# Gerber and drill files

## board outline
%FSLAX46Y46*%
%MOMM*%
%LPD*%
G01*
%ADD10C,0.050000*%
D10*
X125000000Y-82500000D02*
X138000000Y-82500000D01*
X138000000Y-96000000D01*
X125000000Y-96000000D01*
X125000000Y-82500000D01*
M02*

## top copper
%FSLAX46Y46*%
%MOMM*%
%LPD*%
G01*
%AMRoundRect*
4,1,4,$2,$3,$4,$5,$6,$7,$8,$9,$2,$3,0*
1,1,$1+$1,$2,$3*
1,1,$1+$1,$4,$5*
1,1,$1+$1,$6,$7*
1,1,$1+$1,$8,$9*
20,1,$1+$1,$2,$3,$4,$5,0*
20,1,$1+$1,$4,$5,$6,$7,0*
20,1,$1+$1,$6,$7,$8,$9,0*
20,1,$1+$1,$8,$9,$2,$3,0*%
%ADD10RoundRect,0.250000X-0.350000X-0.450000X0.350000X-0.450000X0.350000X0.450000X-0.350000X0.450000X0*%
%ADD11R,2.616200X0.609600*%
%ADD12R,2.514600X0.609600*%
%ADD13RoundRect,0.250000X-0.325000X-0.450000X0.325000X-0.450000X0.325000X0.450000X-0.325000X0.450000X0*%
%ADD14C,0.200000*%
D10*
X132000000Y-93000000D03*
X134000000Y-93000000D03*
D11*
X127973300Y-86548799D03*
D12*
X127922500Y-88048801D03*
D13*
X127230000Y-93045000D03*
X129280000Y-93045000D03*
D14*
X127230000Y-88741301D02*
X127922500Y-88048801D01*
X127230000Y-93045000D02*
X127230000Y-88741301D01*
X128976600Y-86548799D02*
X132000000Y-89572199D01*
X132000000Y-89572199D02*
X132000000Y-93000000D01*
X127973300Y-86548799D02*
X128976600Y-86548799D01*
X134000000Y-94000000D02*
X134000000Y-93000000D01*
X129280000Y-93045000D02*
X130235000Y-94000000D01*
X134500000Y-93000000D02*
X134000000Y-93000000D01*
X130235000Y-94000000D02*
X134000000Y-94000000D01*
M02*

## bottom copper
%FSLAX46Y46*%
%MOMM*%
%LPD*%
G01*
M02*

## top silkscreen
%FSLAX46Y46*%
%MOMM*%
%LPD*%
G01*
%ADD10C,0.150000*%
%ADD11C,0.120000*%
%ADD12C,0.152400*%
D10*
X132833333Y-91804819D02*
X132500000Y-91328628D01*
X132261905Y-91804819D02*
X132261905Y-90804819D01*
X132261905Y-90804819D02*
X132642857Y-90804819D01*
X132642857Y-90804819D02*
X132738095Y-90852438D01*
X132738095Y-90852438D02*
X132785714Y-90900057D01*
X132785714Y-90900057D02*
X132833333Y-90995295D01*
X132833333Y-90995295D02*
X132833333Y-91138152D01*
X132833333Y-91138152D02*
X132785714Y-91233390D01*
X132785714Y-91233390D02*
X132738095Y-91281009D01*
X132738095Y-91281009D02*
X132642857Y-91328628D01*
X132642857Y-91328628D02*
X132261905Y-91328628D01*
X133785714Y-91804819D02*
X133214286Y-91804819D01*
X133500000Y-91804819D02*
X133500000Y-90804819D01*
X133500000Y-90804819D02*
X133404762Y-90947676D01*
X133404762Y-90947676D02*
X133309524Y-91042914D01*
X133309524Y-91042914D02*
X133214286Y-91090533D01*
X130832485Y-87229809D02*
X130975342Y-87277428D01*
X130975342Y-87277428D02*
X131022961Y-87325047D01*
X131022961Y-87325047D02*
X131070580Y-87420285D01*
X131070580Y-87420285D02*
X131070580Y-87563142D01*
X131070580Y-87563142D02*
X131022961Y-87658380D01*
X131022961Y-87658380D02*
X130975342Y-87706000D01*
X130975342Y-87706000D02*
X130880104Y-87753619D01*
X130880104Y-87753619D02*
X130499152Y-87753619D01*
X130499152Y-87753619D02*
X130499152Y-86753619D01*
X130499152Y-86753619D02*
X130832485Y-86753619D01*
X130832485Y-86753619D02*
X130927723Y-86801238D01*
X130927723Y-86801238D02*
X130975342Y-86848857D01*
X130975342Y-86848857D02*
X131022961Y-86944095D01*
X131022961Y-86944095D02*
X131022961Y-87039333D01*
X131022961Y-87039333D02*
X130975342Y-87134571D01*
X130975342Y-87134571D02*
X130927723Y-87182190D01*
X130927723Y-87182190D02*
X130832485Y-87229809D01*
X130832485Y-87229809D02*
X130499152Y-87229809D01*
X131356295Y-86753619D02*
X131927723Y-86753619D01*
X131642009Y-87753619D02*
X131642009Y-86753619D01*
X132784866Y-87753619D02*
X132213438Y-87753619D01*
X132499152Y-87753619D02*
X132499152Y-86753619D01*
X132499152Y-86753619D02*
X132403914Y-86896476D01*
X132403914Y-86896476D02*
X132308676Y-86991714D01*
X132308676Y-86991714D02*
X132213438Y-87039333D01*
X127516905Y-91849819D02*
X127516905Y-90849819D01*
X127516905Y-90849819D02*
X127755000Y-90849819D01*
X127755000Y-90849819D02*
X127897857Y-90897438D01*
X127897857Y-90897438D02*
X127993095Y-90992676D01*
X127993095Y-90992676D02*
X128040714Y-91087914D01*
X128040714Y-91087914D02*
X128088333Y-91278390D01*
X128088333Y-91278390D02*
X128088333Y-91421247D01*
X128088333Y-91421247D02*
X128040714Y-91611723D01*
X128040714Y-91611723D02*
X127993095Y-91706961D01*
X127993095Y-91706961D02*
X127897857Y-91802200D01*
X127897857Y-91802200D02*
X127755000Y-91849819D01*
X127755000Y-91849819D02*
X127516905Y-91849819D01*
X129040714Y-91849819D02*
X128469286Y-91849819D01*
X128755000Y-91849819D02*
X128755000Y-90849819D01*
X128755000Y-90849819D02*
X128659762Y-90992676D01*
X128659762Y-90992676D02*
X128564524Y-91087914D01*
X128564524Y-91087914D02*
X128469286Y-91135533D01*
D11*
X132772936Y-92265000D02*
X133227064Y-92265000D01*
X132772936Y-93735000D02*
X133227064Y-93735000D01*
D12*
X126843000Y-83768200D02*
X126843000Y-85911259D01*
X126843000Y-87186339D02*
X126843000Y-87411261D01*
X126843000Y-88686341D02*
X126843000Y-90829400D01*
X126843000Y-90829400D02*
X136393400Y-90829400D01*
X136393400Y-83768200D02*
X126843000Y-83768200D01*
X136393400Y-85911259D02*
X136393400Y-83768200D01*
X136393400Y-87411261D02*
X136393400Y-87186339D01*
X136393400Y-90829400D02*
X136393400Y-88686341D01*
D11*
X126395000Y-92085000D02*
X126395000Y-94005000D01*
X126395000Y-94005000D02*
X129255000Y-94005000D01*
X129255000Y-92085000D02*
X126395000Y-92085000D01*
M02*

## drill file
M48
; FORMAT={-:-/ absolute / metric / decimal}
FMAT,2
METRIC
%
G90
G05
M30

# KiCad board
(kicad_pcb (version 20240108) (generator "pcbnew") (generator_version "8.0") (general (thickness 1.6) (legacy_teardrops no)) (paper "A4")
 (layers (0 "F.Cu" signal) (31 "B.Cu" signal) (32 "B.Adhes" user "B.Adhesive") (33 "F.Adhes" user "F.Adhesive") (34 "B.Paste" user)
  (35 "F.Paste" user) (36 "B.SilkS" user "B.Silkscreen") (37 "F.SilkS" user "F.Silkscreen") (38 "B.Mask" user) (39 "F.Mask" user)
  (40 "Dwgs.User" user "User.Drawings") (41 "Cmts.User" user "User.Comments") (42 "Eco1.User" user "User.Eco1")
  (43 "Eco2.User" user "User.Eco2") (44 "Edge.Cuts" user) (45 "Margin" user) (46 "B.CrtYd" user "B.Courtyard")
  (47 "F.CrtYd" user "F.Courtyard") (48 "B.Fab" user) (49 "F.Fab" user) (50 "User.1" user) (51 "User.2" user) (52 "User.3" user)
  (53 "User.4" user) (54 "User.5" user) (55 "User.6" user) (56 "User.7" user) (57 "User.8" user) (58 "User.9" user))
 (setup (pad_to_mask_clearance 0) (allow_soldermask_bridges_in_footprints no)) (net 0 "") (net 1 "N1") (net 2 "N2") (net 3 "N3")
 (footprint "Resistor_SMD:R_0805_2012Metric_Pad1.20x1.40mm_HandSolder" (layer "F.Cu") (at 133 93)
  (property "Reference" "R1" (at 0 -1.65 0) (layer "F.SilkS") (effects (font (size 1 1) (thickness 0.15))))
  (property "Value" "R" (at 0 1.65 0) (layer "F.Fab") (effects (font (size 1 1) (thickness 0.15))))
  (fp_line (start -0.227064 -0.735) (end 0.227064 -0.735) (stroke (width 0.12) (type solid)) (layer "F.SilkS"))
  (fp_line (start -0.227064 0.735) (end 0.227064 0.735) (stroke (width 0.12) (type solid)) (layer "F.SilkS"))
  (pad "1" smd roundrect (at -1 0) (size 1.2 1.4) (layers "F.Cu" "F.Paste" "F.Mask") (roundrect_rratio 0.208333) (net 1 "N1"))
  (pad "2" smd roundrect (at 1 0) (size 1.2 1.4) (layers "F.Cu" "F.Paste" "F.Mask") (roundrect_rratio 0.208333) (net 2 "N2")))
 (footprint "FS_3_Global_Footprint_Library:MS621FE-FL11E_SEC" (layer "F.Cu") (at 131.6182 87.2988)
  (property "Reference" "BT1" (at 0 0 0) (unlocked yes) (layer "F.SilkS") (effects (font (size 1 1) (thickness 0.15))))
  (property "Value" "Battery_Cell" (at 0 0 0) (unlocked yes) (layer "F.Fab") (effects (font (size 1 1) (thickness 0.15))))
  (fp_line (start -4.7752 -3.5306) (end -4.7752 -1.387541) (stroke (width 0.1524) (type solid)) (layer "F.SilkS"))
  (fp_line (start -4.7752 -0.112461) (end -4.7752 0.112461) (stroke (width 0.1524) (type solid)) (layer "F.SilkS"))
  (fp_line (start -4.7752 1.387541) (end -4.7752 3.5306) (stroke (width 0.1524) (type solid)) (layer "F.SilkS"))
  (fp_line (start -4.7752 3.5306) (end 4.7752 3.5306) (stroke (width 0.1524) (type solid)) (layer "F.SilkS"))
  (fp_line (start 4.7752 -3.5306) (end -4.7752 -3.5306) (stroke (width 0.1524) (type solid)) (layer "F.SilkS"))
  (fp_line (start 4.7752 -1.387541) (end 4.7752 -3.5306) (stroke (width 0.1524) (type solid)) (layer "F.SilkS"))
  (fp_line (start 4.7752 0.112461) (end 4.7752 -0.112461) (stroke (width 0.1524) (type solid)) (layer "F.SilkS"))
  (fp_line (start 4.7752 3.5306) (end 4.7752 1.387541) (stroke (width 0.1524) (type solid)) (layer "F.SilkS"))
  (pad "1" smd rect (at -3.6449 -0.750001) (size 2.6162 0.6096) (layers "F.Cu" "F.Paste" "F.Mask") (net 1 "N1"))
  (pad "2" smd rect (at -3.6957 0.750001) (size 2.5146 0.6096) (layers "F.Cu" "F.Paste" "F.Mask") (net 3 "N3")))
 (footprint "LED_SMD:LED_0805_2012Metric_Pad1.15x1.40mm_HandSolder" (layer "F.Cu") (at 128.255 93.045)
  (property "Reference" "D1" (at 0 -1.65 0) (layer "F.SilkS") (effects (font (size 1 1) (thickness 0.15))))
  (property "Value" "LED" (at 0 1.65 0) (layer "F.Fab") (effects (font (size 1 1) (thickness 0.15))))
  (fp_line (start -1.86 -0.96) (end -1.86 0.96) (stroke (width 0.12) (type solid)) (layer "F.SilkS"))
  (fp_line (start -1.86 0.96) (end 1 0.96) (stroke (width 0.12) (type solid)) (layer "F.SilkS"))
  (fp_line (start 1 -0.96) (end -1.86 -0.96) (stroke (width 0.12) (type solid)) (layer "F.SilkS"))
  (pad "1" smd roundrect (at -1.025 0) (size 1.15 1.4) (layers "F.Cu" "F.Paste" "F.Mask") (roundrect_rratio 0.217391) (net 3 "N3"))
  (pad "2" smd roundrect (at 1.025 0) (size 1.15 1.4) (layers "F.Cu" "F.Paste" "F.Mask") (roundrect_rratio 0.217391) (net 2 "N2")))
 (gr_rect (start 125 82.5) (end 138 96) (stroke (width 0.05) (type default)) (fill none) (layer "Edge.Cuts"))
 (segment (start 127.23 88.741301) (end 127.9225 88.048801) (width 0.2) (layer "F.Cu") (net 3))
 (segment (start 127.23 93.045) (end 127.23 88.741301) (width 0.2) (layer "F.Cu") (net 3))
 (segment (start 128.9766 86.548799) (end 132 89.572199) (width 0.2) (layer "F.Cu") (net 1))
 (segment (start 132 89.572199) (end 132 93) (width 0.2) (layer "F.Cu") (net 1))
 (segment (start 127.9733 86.548799) (end 128.9766 86.548799) (width 0.2) (layer "F.Cu") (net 1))
 (segment (start 134 94) (end 134 93) (width 0.2) (layer "F.Cu") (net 2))
 (segment (start 129.28 93.045) (end 130.235 94) (width 0.2) (layer "F.Cu") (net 2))
 (segment (start 134.5 93) (end 134 93) (width 0.2) (layer "F.Cu") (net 2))
 (segment (start 130.235 94) (end 134 94) (width 0.2) (layer "F.Cu") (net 2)))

